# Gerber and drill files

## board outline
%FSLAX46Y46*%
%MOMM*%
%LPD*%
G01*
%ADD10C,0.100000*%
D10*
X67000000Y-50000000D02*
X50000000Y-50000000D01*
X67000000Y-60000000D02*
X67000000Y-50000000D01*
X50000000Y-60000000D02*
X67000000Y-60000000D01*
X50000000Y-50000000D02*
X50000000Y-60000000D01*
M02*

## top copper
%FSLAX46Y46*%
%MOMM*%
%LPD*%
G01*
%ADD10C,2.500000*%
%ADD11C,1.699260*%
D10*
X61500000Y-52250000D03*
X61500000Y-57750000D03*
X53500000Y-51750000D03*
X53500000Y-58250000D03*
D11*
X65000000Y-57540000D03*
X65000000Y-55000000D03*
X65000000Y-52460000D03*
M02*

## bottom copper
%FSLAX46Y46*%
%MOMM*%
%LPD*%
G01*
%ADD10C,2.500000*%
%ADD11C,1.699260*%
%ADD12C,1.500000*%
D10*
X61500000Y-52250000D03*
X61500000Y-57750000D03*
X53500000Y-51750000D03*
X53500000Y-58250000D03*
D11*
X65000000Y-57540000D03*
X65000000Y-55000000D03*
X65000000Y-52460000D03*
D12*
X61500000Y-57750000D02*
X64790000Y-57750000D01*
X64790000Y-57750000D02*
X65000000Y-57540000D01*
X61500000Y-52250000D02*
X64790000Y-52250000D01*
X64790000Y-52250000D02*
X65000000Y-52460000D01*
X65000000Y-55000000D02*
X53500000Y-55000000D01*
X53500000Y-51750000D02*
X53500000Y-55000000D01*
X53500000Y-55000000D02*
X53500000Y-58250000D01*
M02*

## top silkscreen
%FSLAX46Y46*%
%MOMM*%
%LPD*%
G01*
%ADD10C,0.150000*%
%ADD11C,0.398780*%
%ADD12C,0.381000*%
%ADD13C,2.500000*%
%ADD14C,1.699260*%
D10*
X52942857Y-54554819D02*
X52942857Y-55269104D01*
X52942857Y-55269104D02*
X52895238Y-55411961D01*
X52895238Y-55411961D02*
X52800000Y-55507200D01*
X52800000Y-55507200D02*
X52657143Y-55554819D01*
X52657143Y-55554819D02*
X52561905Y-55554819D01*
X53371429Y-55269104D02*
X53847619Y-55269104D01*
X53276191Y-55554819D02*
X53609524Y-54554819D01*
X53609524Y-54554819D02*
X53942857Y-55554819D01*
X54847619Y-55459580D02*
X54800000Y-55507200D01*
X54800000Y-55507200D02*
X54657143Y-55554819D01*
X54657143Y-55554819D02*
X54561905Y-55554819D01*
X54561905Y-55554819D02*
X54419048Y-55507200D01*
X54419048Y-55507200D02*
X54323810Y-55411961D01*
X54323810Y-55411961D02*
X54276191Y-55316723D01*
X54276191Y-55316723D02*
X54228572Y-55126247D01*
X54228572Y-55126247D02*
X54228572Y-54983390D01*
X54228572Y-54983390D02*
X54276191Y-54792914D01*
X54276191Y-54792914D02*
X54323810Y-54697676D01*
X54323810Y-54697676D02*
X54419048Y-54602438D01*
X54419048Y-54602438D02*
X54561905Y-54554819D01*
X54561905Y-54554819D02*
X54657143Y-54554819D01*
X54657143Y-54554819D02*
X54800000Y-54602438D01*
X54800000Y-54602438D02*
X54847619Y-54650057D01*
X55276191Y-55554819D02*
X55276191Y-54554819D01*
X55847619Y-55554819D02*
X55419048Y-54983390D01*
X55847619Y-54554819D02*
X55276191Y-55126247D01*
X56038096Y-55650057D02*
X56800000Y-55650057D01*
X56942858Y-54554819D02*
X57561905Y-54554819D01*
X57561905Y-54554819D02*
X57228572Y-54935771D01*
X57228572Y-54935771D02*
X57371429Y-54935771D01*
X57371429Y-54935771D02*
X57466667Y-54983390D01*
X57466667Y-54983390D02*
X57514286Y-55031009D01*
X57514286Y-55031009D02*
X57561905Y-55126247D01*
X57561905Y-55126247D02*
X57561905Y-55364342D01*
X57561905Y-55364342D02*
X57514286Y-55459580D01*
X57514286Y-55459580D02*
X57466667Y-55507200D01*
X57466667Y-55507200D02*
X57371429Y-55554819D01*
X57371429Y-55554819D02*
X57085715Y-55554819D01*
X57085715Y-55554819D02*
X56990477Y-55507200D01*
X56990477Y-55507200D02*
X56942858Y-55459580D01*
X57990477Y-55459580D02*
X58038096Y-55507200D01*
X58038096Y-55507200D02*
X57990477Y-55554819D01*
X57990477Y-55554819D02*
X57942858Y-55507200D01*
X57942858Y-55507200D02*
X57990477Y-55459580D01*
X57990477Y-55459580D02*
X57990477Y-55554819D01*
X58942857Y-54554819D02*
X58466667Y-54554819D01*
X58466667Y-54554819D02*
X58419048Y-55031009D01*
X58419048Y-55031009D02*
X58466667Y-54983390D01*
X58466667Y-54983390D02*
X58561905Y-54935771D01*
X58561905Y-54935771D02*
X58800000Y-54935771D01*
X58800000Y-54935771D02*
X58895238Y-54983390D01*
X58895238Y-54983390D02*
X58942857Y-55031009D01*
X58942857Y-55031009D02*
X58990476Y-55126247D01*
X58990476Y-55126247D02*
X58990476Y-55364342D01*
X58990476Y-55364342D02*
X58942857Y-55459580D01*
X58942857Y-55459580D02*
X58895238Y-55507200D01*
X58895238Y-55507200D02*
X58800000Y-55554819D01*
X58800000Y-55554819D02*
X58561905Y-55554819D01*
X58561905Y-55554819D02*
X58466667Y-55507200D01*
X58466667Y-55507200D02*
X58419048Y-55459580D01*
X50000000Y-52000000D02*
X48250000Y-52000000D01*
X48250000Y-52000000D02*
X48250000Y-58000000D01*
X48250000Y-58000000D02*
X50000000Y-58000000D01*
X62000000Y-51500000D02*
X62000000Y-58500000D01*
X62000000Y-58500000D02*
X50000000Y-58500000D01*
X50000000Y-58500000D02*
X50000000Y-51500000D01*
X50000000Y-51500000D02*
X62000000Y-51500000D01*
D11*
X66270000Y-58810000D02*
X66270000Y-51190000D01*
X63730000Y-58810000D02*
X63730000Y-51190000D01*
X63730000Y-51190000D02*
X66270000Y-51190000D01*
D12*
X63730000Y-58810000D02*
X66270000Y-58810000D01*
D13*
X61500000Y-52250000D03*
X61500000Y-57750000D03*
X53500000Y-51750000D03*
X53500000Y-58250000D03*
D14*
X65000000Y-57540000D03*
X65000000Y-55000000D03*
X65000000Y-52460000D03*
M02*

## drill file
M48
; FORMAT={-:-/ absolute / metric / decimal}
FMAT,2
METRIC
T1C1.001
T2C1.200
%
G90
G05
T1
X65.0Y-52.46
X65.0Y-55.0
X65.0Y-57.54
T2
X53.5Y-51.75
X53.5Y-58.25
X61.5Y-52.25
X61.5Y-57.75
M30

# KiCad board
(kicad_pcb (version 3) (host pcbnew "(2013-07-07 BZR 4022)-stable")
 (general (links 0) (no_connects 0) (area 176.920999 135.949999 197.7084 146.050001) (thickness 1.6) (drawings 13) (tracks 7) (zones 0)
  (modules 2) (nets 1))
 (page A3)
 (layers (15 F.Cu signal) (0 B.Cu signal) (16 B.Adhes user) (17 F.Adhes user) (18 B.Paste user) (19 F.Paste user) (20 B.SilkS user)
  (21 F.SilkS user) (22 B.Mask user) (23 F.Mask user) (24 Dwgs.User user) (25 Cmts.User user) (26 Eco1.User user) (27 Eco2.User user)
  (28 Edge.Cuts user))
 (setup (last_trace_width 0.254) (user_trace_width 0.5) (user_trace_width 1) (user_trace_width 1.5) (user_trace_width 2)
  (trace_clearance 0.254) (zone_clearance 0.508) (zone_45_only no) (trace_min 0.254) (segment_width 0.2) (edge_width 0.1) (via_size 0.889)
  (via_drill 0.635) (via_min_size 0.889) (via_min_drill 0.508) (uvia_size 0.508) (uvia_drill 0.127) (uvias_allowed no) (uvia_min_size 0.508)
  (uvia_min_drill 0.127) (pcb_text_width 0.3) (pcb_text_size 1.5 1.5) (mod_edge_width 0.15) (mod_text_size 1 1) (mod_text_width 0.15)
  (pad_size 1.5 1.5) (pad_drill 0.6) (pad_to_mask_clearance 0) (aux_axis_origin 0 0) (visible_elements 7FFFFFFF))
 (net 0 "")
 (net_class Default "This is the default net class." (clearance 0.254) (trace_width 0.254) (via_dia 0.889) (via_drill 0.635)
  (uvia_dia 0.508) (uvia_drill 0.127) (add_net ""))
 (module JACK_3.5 (layer F.Cu) (at 56 55)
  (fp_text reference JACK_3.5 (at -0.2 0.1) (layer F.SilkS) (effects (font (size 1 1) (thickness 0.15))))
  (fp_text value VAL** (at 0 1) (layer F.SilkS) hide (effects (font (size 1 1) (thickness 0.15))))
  (fp_line (start -6 -3) (end -7.75 -3) (layer F.SilkS) (width 0.15))
  (fp_line (start -7.75 -3) (end -7.75 3) (layer F.SilkS) (width 0.15))
  (fp_line (start -7.75 3) (end -6 3) (layer F.SilkS) (width 0.15))
  (fp_line (start 6 -3.5) (end 6 3.5) (layer F.SilkS) (width 0.15))
  (fp_line (start 6 3.5) (end -6 3.5) (layer F.SilkS) (width 0.15))
  (fp_line (start -6 3.5) (end -6 -3.5) (layer F.SilkS) (width 0.15))
  (fp_line (start -6 -3.5) (end 6 -3.5) (layer F.SilkS) (width 0.15))
  (pad 2 thru_hole circle (at 5.5 -2.75) (size 2.5 2.5) (drill 1.2) (layers *.Cu *.Mask F.SilkS))
  (pad 3 thru_hole circle (at 5.5 2.75) (size 2.5 2.5) (drill 1.2) (layers *.Cu *.Mask F.SilkS))
  (pad 1 thru_hole circle (at -2.5 -3.25) (size 2.5 2.5) (drill 1.2) (layers *.Cu *.Mask F.SilkS))
  (pad 1 thru_hole circle (at -2.5 3.25) (size 2.5 2.5) (drill 1.2) (layers *.Cu *.Mask F.SilkS)))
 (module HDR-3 (layer F.Cu) (at 65 55 90)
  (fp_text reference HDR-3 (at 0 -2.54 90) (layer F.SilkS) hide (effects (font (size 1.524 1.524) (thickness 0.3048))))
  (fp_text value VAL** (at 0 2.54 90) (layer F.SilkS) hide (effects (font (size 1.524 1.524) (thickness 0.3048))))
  (fp_line (start -3.81 1.27) (end 3.81 1.27) (layer F.SilkS) (width 0.39878))
  (fp_line (start -3.81 -1.27) (end 3.81 -1.27) (layer F.SilkS) (width 0.39878))
  (fp_line (start 3.81 -1.27) (end 3.81 1.27) (layer F.SilkS) (width 0.39878))
  (fp_line (start -3.81 -1.27) (end -3.81 1.27) (layer F.SilkS) (width 0.381))
  (pad 1 thru_hole circle (at -2.54 0 90) (size 1.69926 1.69926) (drill 1.00076) (layers *.Cu *.Mask F.SilkS))
  (pad 2 thru_hole circle (at 0 0 90) (size 1.69926 1.69926) (drill 1.00076) (layers *.Cu *.Mask F.SilkS))
  (pad 3 thru_hole circle (at 2.54 0 90) (size 1.69926 1.69926) (drill 1.00076) (layers *.Cu *.Mask F.SilkS)))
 (gr_line (start 67 50) (end 50 50) (angle 90) (layer Edge.Cuts) (width 0.1))
 (gr_line (start 67 60) (end 67 50) (angle 90) (layer Edge.Cuts) (width 0.1))
 (gr_line (start 50 60) (end 67 60) (angle 90) (layer Edge.Cuts) (width 0.1))
 (gr_line (start 50 50) (end 50 60) (angle 90) (layer Edge.Cuts) (width 0.1))
 (segment (start 61.5 57.75) (end 64.79 57.75) (width 1.5) (layer B.Cu) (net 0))
 (segment (start 64.79 57.75) (end 65 57.54) (width 1.5) (layer B.Cu) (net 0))
 (segment (start 61.5 52.25) (end 64.79 52.25) (width 1.5) (layer B.Cu) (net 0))
 (segment (start 64.79 52.25) (end 65 52.46) (width 1.5) (layer B.Cu) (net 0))
 (segment (start 65 55) (end 53.5 55) (width 1.5) (layer B.Cu) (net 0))
 (segment (start 53.5 51.75) (end 53.5 55) (width 1.5) (layer B.Cu) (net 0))
 (segment (start 53.5 55) (end 53.5 58.25) (width 1.5) (layer B.Cu) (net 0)))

